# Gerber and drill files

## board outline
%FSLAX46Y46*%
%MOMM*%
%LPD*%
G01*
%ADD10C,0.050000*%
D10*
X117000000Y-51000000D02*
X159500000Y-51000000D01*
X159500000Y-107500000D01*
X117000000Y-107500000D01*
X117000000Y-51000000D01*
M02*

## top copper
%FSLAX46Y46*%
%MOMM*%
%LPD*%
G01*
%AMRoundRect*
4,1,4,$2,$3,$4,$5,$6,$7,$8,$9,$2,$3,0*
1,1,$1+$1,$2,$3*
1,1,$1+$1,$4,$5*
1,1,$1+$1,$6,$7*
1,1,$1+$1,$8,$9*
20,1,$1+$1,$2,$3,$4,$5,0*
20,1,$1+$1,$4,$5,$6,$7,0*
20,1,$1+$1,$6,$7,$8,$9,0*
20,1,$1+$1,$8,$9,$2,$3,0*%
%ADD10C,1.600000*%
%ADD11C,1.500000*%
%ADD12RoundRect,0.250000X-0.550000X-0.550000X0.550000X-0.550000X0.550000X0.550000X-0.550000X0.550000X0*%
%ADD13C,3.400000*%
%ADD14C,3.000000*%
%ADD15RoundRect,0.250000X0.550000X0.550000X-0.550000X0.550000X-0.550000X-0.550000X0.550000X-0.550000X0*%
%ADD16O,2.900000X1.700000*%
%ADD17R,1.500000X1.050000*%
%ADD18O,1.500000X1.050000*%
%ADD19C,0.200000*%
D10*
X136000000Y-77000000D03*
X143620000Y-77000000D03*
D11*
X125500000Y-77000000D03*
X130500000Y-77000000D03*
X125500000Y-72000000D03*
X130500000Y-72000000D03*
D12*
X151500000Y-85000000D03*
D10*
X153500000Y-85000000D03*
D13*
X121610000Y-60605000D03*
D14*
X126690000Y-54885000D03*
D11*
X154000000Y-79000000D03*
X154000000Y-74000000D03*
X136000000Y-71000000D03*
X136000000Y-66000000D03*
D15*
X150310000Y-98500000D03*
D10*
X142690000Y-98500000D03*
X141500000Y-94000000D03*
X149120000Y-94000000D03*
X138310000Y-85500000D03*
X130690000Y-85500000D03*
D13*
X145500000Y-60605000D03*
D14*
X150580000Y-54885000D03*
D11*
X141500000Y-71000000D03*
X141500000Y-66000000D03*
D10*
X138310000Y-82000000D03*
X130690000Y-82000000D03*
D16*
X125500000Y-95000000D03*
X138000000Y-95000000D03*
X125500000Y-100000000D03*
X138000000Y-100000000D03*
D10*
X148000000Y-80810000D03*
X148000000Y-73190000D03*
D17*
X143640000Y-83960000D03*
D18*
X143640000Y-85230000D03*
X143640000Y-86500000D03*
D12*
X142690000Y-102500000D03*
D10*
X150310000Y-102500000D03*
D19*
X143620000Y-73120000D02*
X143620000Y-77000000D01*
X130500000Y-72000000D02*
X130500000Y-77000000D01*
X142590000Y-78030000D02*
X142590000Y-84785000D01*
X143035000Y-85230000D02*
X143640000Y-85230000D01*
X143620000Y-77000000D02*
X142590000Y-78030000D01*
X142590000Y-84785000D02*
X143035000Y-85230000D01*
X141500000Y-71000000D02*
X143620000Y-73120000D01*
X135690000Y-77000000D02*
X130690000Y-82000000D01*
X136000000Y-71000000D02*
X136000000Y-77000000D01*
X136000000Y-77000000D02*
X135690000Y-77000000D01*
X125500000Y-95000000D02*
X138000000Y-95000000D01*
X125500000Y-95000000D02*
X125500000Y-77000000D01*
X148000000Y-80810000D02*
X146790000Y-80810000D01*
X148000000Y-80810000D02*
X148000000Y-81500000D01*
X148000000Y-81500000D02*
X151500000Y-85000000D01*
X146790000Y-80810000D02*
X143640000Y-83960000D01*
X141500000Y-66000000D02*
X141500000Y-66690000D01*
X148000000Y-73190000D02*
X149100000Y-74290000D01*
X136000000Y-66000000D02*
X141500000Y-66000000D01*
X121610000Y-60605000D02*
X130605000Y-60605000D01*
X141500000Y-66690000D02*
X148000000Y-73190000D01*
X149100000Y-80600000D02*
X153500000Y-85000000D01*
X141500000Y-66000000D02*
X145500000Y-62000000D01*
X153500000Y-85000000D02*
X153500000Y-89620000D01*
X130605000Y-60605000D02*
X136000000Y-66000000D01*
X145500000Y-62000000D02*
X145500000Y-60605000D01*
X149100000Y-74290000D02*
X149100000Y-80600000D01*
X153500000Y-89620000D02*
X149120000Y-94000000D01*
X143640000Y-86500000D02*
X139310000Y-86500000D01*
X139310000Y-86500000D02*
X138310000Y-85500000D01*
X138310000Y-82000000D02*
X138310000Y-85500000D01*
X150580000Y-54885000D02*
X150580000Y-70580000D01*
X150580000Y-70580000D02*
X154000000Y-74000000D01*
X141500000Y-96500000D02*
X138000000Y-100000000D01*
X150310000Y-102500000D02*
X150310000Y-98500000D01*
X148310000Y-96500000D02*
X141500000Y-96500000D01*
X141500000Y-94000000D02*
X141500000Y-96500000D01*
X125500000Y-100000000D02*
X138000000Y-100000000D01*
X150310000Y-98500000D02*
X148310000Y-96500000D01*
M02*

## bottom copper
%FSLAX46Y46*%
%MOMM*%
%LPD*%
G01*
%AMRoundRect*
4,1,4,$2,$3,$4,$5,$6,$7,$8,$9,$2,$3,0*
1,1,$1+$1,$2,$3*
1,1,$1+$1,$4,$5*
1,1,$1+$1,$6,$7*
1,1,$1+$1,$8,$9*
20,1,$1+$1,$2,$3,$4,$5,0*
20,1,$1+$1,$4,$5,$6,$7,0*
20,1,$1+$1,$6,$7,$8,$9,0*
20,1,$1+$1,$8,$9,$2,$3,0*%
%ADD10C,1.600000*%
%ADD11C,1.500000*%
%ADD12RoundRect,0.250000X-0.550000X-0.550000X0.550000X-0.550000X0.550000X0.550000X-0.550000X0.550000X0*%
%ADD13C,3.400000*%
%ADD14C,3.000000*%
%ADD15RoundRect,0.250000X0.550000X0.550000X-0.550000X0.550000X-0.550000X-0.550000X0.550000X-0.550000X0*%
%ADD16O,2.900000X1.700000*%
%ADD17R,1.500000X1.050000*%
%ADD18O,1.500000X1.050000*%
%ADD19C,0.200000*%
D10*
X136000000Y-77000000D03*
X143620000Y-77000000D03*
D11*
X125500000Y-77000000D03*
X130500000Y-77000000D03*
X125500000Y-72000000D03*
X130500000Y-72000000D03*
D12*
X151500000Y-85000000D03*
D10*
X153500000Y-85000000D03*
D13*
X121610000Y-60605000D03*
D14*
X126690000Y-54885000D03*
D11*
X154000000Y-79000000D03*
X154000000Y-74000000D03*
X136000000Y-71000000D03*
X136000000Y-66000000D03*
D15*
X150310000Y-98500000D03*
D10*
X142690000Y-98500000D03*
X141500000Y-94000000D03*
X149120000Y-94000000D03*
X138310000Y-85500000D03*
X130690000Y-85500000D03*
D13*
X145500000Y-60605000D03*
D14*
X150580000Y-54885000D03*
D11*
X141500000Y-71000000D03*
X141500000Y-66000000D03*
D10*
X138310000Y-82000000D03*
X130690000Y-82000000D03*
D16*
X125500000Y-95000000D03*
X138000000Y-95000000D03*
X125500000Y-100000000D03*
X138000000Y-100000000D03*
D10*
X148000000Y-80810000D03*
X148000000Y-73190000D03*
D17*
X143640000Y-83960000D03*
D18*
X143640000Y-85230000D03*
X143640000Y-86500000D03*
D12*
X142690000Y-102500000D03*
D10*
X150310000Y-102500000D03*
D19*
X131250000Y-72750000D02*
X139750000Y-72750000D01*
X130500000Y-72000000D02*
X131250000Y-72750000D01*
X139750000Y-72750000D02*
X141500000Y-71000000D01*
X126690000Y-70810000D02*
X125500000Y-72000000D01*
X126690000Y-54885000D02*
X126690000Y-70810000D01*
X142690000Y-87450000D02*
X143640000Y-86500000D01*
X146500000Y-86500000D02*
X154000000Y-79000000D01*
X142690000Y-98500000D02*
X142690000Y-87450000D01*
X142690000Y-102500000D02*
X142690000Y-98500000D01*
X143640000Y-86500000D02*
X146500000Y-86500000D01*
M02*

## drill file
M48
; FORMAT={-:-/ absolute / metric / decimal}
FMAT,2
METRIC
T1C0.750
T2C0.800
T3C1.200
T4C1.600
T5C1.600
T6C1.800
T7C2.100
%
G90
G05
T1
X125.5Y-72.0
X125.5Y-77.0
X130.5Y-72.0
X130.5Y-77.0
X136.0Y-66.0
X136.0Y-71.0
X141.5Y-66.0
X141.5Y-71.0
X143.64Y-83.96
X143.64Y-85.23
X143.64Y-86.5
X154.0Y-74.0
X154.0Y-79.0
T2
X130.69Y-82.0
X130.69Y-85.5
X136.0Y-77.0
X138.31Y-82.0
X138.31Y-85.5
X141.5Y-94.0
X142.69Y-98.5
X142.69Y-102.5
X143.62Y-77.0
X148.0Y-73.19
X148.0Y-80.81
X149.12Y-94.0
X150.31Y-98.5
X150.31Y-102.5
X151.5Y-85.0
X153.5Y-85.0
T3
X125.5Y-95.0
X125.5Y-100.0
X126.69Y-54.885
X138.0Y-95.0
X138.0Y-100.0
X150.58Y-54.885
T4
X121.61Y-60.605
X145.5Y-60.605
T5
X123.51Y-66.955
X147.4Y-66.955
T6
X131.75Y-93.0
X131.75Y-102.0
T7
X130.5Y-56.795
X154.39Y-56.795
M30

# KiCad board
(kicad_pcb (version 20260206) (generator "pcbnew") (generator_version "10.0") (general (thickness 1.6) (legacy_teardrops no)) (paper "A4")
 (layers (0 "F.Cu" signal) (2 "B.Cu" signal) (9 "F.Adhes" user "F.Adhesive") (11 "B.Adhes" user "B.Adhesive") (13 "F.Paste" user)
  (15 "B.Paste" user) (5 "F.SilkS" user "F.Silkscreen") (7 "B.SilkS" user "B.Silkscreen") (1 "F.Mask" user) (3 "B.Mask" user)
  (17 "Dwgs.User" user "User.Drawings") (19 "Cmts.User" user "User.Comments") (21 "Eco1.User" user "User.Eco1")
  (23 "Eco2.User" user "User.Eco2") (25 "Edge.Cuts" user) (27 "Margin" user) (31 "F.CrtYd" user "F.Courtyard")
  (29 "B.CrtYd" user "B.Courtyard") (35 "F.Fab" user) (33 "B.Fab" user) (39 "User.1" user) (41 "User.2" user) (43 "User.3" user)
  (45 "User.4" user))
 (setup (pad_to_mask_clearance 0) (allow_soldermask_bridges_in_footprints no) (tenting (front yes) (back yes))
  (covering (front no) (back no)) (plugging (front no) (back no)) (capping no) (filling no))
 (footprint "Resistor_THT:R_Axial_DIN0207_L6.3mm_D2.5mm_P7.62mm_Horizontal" (layer "F.Cu") (at 136 77)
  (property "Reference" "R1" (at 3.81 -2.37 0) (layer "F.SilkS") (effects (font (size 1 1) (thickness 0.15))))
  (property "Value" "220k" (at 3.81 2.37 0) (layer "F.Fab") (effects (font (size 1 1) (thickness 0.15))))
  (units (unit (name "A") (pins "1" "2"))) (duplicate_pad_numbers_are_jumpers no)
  (pad "1" thru_hole circle (at 0 0) (size 1.6 1.6) (drill 0.8) (layers "*.Cu" "*.Mask") (remove_unused_layers no) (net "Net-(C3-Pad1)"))
  (pad "2" thru_hole circle (at 7.62 0) (size 1.6 1.6) (drill 0.8) (layers "*.Cu" "*.Mask") (remove_unused_layers no) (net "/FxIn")))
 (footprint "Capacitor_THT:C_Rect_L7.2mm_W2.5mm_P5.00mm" (layer "F.Cu") (at 125.5 77)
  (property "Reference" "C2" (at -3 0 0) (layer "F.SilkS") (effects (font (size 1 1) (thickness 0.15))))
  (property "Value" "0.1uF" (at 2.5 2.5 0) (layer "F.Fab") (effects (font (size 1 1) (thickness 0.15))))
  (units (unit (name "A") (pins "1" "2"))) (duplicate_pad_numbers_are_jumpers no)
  (pad "1" thru_hole circle (at 0 0) (size 1.5 1.5) (drill 0.75) (layers "*.Cu" "*.Mask") (remove_unused_layers no) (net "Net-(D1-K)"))
  (pad "2" thru_hole circle (at 5 0) (size 1.5 1.5) (drill 0.75) (layers "*.Cu" "*.Mask") (remove_unused_layers no) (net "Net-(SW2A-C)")))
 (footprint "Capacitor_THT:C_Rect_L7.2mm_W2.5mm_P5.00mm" (layer "F.Cu") (at 125.5 72)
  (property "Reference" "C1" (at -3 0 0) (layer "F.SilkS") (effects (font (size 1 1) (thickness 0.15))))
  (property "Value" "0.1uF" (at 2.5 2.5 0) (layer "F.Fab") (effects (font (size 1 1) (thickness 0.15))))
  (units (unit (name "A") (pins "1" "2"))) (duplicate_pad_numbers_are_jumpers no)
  (pad "1" thru_hole circle (at 0 0) (size 1.5 1.5) (drill 0.75) (layers "*.Cu" "*.Mask") (remove_unused_layers no) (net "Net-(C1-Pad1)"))
  (pad "2" thru_hole circle (at 5 0) (size 1.5 1.5) (drill 0.75) (layers "*.Cu" "*.Mask") (remove_unused_layers no) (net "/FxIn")))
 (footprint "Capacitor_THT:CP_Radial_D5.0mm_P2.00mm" (layer "F.Cu") (at 151.5 85)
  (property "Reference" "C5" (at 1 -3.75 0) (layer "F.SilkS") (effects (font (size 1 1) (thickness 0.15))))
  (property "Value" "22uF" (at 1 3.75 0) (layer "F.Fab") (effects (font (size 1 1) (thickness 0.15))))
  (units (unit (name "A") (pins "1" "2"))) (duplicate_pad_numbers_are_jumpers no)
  (pad "1" thru_hole roundrect (at 0 0) (size 1.6 1.6) (drill 0.8) (layers "*.Cu" "*.Mask") (remove_unused_layers no)
   (roundrect_rratio 0.15625) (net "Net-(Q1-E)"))
  (pad "2" thru_hole circle (at 2 0) (size 1.6 1.6) (drill 0.8) (layers "*.Cu" "*.Mask") (remove_unused_layers no) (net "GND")))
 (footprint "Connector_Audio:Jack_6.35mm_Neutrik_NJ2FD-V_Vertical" (layer "F.Cu") (at 126.69 54.885)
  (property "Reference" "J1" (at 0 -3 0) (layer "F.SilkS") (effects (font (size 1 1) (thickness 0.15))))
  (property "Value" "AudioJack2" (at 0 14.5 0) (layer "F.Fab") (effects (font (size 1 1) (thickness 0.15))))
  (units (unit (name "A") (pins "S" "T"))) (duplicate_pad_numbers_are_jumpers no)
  (pad "" np_thru_hole circle (at -3.18 12.07 180) (size 1.6 1.6) (drill 1.6) (layers "*.Cu" "*.Mask"))
  (pad "" np_thru_hole circle (at 3.81 1.91 180) (size 2.1 2.1) (drill 2.1) (layers "*.Cu" "*.Mask"))
  (pad "S" thru_hole circle (at -5.08 5.72 180) (size 3.4 3.4) (drill 1.6) (layers "*.Cu" "*.Mask") (remove_unused_layers no) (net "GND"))
  (pad "T" thru_hole circle (at 0 0 180) (size 3 3) (drill 1.2) (layers "*.Cu" "*.Mask") (remove_unused_layers no) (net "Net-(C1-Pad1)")))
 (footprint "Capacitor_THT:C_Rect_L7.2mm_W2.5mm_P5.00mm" (layer "F.Cu") (at 154 79 90)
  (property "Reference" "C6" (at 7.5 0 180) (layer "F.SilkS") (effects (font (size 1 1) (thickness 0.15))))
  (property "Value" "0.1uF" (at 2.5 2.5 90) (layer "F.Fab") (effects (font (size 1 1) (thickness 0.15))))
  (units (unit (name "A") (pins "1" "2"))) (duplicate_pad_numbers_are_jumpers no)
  (pad "1" thru_hole circle (at 0 0 90) (size 1.5 1.5) (drill 0.75) (layers "*.Cu" "*.Mask") (remove_unused_layers no) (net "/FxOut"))
  (pad "2" thru_hole circle (at 5 0 90) (size 1.5 1.5) (drill 0.75) (layers "*.Cu" "*.Mask") (remove_unused_layers no) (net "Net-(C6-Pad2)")))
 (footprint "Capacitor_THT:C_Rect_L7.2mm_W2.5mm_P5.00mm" (layer "F.Cu") (at 136 71 90)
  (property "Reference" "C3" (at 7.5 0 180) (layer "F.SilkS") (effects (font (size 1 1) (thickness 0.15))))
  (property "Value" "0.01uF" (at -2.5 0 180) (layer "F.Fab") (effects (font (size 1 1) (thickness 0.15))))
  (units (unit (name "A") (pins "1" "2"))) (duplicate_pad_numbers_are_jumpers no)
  (pad "1" thru_hole circle (at 0 0 90) (size 1.5 1.5) (drill 0.75) (layers "*.Cu" "*.Mask") (remove_unused_layers no) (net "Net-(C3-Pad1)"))
  (pad "2" thru_hole circle (at 5 0 90) (size 1.5 1.5) (drill 0.75) (layers "*.Cu" "*.Mask") (remove_unused_layers no) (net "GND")))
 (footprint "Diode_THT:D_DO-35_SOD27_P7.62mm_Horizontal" (layer "F.Cu") (at 150.31 98.5 180)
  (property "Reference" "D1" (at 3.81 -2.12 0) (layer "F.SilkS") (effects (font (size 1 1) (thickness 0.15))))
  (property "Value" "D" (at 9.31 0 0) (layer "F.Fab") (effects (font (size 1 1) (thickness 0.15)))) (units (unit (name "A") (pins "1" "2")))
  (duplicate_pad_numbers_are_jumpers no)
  (pad "1" thru_hole roundrect (at 0 0 180) (size 1.6 1.6) (drill 0.8) (layers "*.Cu" "*.Mask") (remove_unused_layers no)
   (roundrect_rratio 0.15625) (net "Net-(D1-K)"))
  (pad "2" thru_hole circle (at 7.62 0 180) (size 1.6 1.6) (drill 0.8) (layers "*.Cu" "*.Mask") (remove_unused_layers no) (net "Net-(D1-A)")))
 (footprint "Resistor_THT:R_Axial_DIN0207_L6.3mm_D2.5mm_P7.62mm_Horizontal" (layer "F.Cu") (at 141.5 94)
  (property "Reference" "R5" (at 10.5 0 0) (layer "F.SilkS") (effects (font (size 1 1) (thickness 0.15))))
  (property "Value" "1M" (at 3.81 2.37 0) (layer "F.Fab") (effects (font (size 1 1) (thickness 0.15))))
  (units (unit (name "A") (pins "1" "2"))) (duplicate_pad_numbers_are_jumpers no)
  (pad "1" thru_hole circle (at 0 0) (size 1.6 1.6) (drill 0.8) (layers "*.Cu" "*.Mask") (remove_unused_layers no) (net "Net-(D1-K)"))
  (pad "2" thru_hole circle (at 7.62 0) (size 1.6 1.6) (drill 0.8) (layers "*.Cu" "*.Mask") (remove_unused_layers no) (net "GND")))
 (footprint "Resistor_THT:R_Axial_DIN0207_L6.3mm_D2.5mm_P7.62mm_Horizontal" (layer "F.Cu") (at 138.31 85.5 180)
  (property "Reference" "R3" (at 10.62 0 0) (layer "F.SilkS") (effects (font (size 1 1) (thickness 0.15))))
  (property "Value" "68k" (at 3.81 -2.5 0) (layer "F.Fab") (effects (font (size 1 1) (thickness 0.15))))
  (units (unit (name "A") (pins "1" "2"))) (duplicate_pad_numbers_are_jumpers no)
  (pad "1" thru_hole circle (at 0 0 180) (size 1.6 1.6) (drill 0.8) (layers "*.Cu" "*.Mask") (remove_unused_layers no) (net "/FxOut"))
  (pad "2" thru_hole circle (at 7.62 0 180) (size 1.6 1.6) (drill 0.8) (layers "*.Cu" "*.Mask") (remove_unused_layers no) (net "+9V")))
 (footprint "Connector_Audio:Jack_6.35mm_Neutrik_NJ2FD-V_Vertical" (layer "F.Cu") (at 150.58 54.885)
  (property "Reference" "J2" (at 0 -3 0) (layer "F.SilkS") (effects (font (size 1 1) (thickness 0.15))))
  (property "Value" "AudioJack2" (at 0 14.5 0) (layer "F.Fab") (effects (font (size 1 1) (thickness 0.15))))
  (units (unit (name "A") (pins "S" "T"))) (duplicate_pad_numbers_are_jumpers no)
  (pad "" np_thru_hole circle (at -3.18 12.07 180) (size 1.6 1.6) (drill 1.6) (layers "*.Cu" "*.Mask"))
  (pad "" np_thru_hole circle (at 3.81 1.91 180) (size 2.1 2.1) (drill 2.1) (layers "*.Cu" "*.Mask"))
  (pad "S" thru_hole circle (at -5.08 5.72 180) (size 3.4 3.4) (drill 1.6) (layers "*.Cu" "*.Mask") (remove_unused_layers no) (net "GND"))
  (pad "T" thru_hole circle (at 0 0 180) (size 3 3) (drill 1.2) (layers "*.Cu" "*.Mask") (remove_unused_layers no) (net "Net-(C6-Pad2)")))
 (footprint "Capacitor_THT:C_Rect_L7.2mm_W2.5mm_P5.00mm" (layer "F.Cu") (at 141.5 71 90)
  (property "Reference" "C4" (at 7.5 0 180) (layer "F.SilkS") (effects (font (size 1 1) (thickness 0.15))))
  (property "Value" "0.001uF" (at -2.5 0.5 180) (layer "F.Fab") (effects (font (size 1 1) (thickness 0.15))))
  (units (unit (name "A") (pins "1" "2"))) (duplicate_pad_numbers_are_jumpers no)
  (pad "1" thru_hole circle (at 0 0 90) (size 1.5 1.5) (drill 0.75) (layers "*.Cu" "*.Mask") (remove_unused_layers no) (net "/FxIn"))
  (pad "2" thru_hole circle (at 5 0 90) (size 1.5 1.5) (drill 0.75) (layers "*.Cu" "*.Mask") (remove_unused_layers no) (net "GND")))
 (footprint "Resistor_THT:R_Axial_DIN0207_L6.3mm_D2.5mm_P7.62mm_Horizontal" (layer "F.Cu") (at 138.31 82 180)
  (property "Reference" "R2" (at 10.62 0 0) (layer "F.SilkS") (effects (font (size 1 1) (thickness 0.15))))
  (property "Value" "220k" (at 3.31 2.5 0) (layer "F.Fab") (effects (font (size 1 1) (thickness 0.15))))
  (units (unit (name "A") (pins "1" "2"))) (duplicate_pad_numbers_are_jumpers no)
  (pad "1" thru_hole circle (at 0 0 180) (size 1.6 1.6) (drill 0.8) (layers "*.Cu" "*.Mask") (remove_unused_layers no) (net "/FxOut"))
  (pad "2" thru_hole circle (at 7.62 0 180) (size 1.6 1.6) (drill 0.8) (layers "*.Cu" "*.Mask") (remove_unused_layers no)
   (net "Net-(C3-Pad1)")))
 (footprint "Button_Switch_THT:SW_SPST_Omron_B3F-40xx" (layer "F.Cu") (at 125.5 95)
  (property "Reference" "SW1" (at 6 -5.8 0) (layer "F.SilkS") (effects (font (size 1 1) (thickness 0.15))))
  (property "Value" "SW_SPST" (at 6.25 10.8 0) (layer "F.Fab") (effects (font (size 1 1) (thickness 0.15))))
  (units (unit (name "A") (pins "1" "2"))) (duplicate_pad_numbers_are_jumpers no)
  (pad "" np_thru_hole circle (at 6.25 -2) (size 1.8 1.8) (drill 1.8) (layers "*.Cu" "*.Mask"))
  (pad "" np_thru_hole circle (at 6.25 7) (size 1.8 1.8) (drill 1.8) (layers "*.Cu" "*.Mask"))
  (pad "1" thru_hole oval (at 0 0) (size 2.9 1.7) (drill 1.2) (layers "*.Cu" "*.Mask") (remove_unused_layers no) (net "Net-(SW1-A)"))
  (pad "1" thru_hole oval (at 12.5 0) (size 2.9 1.7) (drill 1.2) (layers "*.Cu" "*.Mask") (remove_unused_layers no) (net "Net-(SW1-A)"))
  (pad "2" thru_hole oval (at 0 5) (size 2.9 1.7) (drill 1.2) (layers "*.Cu" "*.Mask") (remove_unused_layers no) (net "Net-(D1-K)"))
  (pad "2" thru_hole oval (at 12.5 5) (size 2.9 1.7) (drill 1.2) (layers "*.Cu" "*.Mask") (remove_unused_layers no) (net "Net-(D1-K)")))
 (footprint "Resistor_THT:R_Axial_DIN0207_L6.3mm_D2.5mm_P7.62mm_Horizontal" (layer "F.Cu") (at 148 80.81 90)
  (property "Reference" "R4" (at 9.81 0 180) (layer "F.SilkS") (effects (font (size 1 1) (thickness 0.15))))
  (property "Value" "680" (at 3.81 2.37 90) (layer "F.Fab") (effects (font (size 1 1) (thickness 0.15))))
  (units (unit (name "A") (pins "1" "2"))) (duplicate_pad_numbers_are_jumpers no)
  (pad "1" thru_hole circle (at 0 0 90) (size 1.6 1.6) (drill 0.8) (layers "*.Cu" "*.Mask") (remove_unused_layers no) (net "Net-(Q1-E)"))
  (pad "2" thru_hole circle (at 7.62 0 90) (size 1.6 1.6) (drill 0.8) (layers "*.Cu" "*.Mask") (remove_unused_layers no) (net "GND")))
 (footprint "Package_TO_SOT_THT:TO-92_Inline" (layer "F.Cu") (at 143.64 83.96 -90)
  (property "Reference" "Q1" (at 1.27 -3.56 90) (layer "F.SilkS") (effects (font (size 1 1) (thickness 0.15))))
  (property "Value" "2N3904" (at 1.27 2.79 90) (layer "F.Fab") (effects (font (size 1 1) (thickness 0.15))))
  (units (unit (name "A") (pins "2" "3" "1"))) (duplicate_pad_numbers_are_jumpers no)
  (pad "1" thru_hole rect (at 0 0 270) (size 1.05 1.5) (drill 0.75) (layers "*.Cu" "*.Mask") (remove_unused_layers no) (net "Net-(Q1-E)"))
  (pad "2" thru_hole oval (at 1.27 0 270) (size 1.05 1.5) (drill 0.75) (layers "*.Cu" "*.Mask") (remove_unused_layers no) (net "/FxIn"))
  (pad "3" thru_hole oval (at 2.54 0 270) (size 1.05 1.5) (drill 0.75) (layers "*.Cu" "*.Mask") (remove_unused_layers no) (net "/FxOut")))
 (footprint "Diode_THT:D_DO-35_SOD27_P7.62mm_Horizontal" (layer "F.Cu") (at 142.69 102.5)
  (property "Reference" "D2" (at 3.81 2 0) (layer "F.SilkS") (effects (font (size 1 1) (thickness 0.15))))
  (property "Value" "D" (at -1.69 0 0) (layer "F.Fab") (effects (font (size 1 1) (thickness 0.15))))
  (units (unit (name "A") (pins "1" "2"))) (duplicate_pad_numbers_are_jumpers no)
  (pad "1" thru_hole roundrect (at 0 0) (size 1.6 1.6) (drill 0.8) (layers "*.Cu" "*.Mask") (remove_unused_layers no)
   (roundrect_rratio 0.15625) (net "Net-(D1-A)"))
  (pad "2" thru_hole circle (at 7.62 0) (size 1.6 1.6) (drill 0.8) (layers "*.Cu" "*.Mask") (remove_unused_layers no) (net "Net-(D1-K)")))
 (gr_rect (start 117 51) (end 159.5 107.5) (stroke (width 0.05) (type default)) (fill no) (layer "Edge.Cuts"))
 (segment (start 143.62 73.12) (end 143.62 77) (width 0.2) (layer "F.Cu") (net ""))
 (segment (start 130.5 72) (end 130.5 77) (width 0.2) (layer "F.Cu") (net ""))
 (segment (start 142.59 78.03) (end 142.59 84.785) (width 0.2) (layer "F.Cu") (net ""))
 (segment (start 143.035 85.23) (end 143.64 85.23) (width 0.2) (layer "F.Cu") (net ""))
 (segment (start 143.62 77) (end 142.59 78.03) (width 0.2) (layer "F.Cu") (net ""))
 (segment (start 142.59 84.785) (end 143.035 85.23) (width 0.2) (layer "F.Cu") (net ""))
 (segment (start 141.5 71) (end 143.62 73.12) (width 0.2) (layer "F.Cu") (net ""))
 (segment (start 131.25 72.75) (end 139.75 72.75) (width 0.2) (layer "B.Cu") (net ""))
 (segment (start 130.5 72) (end 131.25 72.75) (width 0.2) (layer "B.Cu") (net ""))
 (segment (start 139.75 72.75) (end 141.5 71) (width 0.2) (layer "B.Cu") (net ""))
 (segment (start 135.69 77) (end 130.69 82) (width 0.2) (layer "F.Cu") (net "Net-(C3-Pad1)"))
 (segment (start 136 71) (end 136 77) (width 0.2) (layer "F.Cu") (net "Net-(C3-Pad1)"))
 (segment (start 136 77) (end 135.69 77) (width 0.2) (layer "F.Cu") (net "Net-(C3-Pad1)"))
 (segment (start 125.5 95) (end 138 95) (width 0.2) (layer "F.Cu") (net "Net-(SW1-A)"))
 (segment (start 125.5 95) (end 125.5 77) (width 0.2) (layer "F.Cu") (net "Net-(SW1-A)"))
 (segment (start 126.69 70.81) (end 125.5 72) (width 0.2) (layer "B.Cu") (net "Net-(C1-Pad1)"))
 (segment (start 126.69 54.885) (end 126.69 70.81) (width 0.2) (layer "B.Cu") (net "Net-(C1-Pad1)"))
 (segment (start 148 80.81) (end 146.79 80.81) (width 0.2) (layer "F.Cu") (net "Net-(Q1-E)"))
 (segment (start 148 80.81) (end 148 81.5) (width 0.2) (layer "F.Cu") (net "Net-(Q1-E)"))
 (segment (start 148 81.5) (end 151.5 85) (width 0.2) (layer "F.Cu") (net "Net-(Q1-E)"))
 (segment (start 146.79 80.81) (end 143.64 83.96) (width 0.2) (layer "F.Cu") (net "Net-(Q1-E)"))
 (segment (start 141.5 66) (end 141.5 66.69) (width 0.2) (layer "F.Cu") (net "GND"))
 (segment (start 148 73.19) (end 149.1 74.29) (width 0.2) (layer "F.Cu") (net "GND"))
 (segment (start 136 66) (end 141.5 66) (width 0.2) (layer "F.Cu") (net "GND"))
 (segment (start 121.61 60.605) (end 130.605 60.605) (width 0.2) (layer "F.Cu") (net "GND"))
 (segment (start 141.5 66.69) (end 148 73.19) (width 0.2) (layer "F.Cu") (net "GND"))
 (segment (start 149.1 80.6) (end 153.5 85) (width 0.2) (layer "F.Cu") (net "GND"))
 (segment (start 141.5 66) (end 145.5 62) (width 0.2) (layer "F.Cu") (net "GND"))
 (segment (start 153.5 85) (end 153.5 89.62) (width 0.2) (layer "F.Cu") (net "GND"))
 (segment (start 130.605 60.605) (end 136 66) (width 0.2) (layer "F.Cu") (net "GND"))
 (segment (start 145.5 62) (end 145.5 60.605) (width 0.2) (layer "F.Cu") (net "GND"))
 (segment (start 149.1 74.29) (end 149.1 80.6) (width 0.2) (layer "F.Cu") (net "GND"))
 (segment (start 153.5 89.62) (end 149.12 94) (width 0.2) (layer "F.Cu") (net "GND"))
 (segment (start 143.64 86.5) (end 139.31 86.5) (width 0.2) (layer "F.Cu") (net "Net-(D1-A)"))
 (segment (start 139.31 86.5) (end 138.31 85.5) (width 0.2) (layer "F.Cu") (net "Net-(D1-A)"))
 (segment (start 138.31 82) (end 138.31 85.5) (width 0.2) (layer "F.Cu") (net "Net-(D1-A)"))
 (segment (start 142.69 87.45) (end 143.64 86.5) (width 0.2) (layer "B.Cu") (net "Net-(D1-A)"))
 (segment (start 146.5 86.5) (end 154 79) (width 0.2) (layer "B.Cu") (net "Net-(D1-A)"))
 (segment (start 142.69 98.5) (end 142.69 87.45) (width 0.2) (layer "B.Cu") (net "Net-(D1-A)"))
 (segment (start 142.69 102.5) (end 142.69 98.5) (width 0.2) (layer "B.Cu") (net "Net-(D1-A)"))
 (segment (start 143.64 86.5) (end 146.5 86.5) (width 0.2) (layer "B.Cu") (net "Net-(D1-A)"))
 (segment (start 150.58 54.885) (end 150.58 70.58) (width 0.2) (layer "F.Cu") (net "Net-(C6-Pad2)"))
 (segment (start 150.58 70.58) (end 154 74) (width 0.2) (layer "F.Cu") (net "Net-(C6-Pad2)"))
 (segment (start 141.5 96.5) (end 138 100) (width 0.2) (layer "F.Cu") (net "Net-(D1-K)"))
 (segment (start 150.31 102.5) (end 150.31 98.5) (width 0.2) (layer "F.Cu") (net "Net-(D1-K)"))
 (segment (start 148.31 96.5) (end 141.5 96.5) (width 0.2) (layer "F.Cu") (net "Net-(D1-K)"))
 (segment (start 141.5 94) (end 141.5 96.5) (width 0.2) (layer "F.Cu") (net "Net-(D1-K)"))
 (segment (start 125.5 100) (end 138 100) (width 0.2) (layer "F.Cu") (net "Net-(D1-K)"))
 (segment (start 150.31 98.5) (end 148.31 96.5) (width 0.2) (layer "F.Cu") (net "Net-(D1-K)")))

